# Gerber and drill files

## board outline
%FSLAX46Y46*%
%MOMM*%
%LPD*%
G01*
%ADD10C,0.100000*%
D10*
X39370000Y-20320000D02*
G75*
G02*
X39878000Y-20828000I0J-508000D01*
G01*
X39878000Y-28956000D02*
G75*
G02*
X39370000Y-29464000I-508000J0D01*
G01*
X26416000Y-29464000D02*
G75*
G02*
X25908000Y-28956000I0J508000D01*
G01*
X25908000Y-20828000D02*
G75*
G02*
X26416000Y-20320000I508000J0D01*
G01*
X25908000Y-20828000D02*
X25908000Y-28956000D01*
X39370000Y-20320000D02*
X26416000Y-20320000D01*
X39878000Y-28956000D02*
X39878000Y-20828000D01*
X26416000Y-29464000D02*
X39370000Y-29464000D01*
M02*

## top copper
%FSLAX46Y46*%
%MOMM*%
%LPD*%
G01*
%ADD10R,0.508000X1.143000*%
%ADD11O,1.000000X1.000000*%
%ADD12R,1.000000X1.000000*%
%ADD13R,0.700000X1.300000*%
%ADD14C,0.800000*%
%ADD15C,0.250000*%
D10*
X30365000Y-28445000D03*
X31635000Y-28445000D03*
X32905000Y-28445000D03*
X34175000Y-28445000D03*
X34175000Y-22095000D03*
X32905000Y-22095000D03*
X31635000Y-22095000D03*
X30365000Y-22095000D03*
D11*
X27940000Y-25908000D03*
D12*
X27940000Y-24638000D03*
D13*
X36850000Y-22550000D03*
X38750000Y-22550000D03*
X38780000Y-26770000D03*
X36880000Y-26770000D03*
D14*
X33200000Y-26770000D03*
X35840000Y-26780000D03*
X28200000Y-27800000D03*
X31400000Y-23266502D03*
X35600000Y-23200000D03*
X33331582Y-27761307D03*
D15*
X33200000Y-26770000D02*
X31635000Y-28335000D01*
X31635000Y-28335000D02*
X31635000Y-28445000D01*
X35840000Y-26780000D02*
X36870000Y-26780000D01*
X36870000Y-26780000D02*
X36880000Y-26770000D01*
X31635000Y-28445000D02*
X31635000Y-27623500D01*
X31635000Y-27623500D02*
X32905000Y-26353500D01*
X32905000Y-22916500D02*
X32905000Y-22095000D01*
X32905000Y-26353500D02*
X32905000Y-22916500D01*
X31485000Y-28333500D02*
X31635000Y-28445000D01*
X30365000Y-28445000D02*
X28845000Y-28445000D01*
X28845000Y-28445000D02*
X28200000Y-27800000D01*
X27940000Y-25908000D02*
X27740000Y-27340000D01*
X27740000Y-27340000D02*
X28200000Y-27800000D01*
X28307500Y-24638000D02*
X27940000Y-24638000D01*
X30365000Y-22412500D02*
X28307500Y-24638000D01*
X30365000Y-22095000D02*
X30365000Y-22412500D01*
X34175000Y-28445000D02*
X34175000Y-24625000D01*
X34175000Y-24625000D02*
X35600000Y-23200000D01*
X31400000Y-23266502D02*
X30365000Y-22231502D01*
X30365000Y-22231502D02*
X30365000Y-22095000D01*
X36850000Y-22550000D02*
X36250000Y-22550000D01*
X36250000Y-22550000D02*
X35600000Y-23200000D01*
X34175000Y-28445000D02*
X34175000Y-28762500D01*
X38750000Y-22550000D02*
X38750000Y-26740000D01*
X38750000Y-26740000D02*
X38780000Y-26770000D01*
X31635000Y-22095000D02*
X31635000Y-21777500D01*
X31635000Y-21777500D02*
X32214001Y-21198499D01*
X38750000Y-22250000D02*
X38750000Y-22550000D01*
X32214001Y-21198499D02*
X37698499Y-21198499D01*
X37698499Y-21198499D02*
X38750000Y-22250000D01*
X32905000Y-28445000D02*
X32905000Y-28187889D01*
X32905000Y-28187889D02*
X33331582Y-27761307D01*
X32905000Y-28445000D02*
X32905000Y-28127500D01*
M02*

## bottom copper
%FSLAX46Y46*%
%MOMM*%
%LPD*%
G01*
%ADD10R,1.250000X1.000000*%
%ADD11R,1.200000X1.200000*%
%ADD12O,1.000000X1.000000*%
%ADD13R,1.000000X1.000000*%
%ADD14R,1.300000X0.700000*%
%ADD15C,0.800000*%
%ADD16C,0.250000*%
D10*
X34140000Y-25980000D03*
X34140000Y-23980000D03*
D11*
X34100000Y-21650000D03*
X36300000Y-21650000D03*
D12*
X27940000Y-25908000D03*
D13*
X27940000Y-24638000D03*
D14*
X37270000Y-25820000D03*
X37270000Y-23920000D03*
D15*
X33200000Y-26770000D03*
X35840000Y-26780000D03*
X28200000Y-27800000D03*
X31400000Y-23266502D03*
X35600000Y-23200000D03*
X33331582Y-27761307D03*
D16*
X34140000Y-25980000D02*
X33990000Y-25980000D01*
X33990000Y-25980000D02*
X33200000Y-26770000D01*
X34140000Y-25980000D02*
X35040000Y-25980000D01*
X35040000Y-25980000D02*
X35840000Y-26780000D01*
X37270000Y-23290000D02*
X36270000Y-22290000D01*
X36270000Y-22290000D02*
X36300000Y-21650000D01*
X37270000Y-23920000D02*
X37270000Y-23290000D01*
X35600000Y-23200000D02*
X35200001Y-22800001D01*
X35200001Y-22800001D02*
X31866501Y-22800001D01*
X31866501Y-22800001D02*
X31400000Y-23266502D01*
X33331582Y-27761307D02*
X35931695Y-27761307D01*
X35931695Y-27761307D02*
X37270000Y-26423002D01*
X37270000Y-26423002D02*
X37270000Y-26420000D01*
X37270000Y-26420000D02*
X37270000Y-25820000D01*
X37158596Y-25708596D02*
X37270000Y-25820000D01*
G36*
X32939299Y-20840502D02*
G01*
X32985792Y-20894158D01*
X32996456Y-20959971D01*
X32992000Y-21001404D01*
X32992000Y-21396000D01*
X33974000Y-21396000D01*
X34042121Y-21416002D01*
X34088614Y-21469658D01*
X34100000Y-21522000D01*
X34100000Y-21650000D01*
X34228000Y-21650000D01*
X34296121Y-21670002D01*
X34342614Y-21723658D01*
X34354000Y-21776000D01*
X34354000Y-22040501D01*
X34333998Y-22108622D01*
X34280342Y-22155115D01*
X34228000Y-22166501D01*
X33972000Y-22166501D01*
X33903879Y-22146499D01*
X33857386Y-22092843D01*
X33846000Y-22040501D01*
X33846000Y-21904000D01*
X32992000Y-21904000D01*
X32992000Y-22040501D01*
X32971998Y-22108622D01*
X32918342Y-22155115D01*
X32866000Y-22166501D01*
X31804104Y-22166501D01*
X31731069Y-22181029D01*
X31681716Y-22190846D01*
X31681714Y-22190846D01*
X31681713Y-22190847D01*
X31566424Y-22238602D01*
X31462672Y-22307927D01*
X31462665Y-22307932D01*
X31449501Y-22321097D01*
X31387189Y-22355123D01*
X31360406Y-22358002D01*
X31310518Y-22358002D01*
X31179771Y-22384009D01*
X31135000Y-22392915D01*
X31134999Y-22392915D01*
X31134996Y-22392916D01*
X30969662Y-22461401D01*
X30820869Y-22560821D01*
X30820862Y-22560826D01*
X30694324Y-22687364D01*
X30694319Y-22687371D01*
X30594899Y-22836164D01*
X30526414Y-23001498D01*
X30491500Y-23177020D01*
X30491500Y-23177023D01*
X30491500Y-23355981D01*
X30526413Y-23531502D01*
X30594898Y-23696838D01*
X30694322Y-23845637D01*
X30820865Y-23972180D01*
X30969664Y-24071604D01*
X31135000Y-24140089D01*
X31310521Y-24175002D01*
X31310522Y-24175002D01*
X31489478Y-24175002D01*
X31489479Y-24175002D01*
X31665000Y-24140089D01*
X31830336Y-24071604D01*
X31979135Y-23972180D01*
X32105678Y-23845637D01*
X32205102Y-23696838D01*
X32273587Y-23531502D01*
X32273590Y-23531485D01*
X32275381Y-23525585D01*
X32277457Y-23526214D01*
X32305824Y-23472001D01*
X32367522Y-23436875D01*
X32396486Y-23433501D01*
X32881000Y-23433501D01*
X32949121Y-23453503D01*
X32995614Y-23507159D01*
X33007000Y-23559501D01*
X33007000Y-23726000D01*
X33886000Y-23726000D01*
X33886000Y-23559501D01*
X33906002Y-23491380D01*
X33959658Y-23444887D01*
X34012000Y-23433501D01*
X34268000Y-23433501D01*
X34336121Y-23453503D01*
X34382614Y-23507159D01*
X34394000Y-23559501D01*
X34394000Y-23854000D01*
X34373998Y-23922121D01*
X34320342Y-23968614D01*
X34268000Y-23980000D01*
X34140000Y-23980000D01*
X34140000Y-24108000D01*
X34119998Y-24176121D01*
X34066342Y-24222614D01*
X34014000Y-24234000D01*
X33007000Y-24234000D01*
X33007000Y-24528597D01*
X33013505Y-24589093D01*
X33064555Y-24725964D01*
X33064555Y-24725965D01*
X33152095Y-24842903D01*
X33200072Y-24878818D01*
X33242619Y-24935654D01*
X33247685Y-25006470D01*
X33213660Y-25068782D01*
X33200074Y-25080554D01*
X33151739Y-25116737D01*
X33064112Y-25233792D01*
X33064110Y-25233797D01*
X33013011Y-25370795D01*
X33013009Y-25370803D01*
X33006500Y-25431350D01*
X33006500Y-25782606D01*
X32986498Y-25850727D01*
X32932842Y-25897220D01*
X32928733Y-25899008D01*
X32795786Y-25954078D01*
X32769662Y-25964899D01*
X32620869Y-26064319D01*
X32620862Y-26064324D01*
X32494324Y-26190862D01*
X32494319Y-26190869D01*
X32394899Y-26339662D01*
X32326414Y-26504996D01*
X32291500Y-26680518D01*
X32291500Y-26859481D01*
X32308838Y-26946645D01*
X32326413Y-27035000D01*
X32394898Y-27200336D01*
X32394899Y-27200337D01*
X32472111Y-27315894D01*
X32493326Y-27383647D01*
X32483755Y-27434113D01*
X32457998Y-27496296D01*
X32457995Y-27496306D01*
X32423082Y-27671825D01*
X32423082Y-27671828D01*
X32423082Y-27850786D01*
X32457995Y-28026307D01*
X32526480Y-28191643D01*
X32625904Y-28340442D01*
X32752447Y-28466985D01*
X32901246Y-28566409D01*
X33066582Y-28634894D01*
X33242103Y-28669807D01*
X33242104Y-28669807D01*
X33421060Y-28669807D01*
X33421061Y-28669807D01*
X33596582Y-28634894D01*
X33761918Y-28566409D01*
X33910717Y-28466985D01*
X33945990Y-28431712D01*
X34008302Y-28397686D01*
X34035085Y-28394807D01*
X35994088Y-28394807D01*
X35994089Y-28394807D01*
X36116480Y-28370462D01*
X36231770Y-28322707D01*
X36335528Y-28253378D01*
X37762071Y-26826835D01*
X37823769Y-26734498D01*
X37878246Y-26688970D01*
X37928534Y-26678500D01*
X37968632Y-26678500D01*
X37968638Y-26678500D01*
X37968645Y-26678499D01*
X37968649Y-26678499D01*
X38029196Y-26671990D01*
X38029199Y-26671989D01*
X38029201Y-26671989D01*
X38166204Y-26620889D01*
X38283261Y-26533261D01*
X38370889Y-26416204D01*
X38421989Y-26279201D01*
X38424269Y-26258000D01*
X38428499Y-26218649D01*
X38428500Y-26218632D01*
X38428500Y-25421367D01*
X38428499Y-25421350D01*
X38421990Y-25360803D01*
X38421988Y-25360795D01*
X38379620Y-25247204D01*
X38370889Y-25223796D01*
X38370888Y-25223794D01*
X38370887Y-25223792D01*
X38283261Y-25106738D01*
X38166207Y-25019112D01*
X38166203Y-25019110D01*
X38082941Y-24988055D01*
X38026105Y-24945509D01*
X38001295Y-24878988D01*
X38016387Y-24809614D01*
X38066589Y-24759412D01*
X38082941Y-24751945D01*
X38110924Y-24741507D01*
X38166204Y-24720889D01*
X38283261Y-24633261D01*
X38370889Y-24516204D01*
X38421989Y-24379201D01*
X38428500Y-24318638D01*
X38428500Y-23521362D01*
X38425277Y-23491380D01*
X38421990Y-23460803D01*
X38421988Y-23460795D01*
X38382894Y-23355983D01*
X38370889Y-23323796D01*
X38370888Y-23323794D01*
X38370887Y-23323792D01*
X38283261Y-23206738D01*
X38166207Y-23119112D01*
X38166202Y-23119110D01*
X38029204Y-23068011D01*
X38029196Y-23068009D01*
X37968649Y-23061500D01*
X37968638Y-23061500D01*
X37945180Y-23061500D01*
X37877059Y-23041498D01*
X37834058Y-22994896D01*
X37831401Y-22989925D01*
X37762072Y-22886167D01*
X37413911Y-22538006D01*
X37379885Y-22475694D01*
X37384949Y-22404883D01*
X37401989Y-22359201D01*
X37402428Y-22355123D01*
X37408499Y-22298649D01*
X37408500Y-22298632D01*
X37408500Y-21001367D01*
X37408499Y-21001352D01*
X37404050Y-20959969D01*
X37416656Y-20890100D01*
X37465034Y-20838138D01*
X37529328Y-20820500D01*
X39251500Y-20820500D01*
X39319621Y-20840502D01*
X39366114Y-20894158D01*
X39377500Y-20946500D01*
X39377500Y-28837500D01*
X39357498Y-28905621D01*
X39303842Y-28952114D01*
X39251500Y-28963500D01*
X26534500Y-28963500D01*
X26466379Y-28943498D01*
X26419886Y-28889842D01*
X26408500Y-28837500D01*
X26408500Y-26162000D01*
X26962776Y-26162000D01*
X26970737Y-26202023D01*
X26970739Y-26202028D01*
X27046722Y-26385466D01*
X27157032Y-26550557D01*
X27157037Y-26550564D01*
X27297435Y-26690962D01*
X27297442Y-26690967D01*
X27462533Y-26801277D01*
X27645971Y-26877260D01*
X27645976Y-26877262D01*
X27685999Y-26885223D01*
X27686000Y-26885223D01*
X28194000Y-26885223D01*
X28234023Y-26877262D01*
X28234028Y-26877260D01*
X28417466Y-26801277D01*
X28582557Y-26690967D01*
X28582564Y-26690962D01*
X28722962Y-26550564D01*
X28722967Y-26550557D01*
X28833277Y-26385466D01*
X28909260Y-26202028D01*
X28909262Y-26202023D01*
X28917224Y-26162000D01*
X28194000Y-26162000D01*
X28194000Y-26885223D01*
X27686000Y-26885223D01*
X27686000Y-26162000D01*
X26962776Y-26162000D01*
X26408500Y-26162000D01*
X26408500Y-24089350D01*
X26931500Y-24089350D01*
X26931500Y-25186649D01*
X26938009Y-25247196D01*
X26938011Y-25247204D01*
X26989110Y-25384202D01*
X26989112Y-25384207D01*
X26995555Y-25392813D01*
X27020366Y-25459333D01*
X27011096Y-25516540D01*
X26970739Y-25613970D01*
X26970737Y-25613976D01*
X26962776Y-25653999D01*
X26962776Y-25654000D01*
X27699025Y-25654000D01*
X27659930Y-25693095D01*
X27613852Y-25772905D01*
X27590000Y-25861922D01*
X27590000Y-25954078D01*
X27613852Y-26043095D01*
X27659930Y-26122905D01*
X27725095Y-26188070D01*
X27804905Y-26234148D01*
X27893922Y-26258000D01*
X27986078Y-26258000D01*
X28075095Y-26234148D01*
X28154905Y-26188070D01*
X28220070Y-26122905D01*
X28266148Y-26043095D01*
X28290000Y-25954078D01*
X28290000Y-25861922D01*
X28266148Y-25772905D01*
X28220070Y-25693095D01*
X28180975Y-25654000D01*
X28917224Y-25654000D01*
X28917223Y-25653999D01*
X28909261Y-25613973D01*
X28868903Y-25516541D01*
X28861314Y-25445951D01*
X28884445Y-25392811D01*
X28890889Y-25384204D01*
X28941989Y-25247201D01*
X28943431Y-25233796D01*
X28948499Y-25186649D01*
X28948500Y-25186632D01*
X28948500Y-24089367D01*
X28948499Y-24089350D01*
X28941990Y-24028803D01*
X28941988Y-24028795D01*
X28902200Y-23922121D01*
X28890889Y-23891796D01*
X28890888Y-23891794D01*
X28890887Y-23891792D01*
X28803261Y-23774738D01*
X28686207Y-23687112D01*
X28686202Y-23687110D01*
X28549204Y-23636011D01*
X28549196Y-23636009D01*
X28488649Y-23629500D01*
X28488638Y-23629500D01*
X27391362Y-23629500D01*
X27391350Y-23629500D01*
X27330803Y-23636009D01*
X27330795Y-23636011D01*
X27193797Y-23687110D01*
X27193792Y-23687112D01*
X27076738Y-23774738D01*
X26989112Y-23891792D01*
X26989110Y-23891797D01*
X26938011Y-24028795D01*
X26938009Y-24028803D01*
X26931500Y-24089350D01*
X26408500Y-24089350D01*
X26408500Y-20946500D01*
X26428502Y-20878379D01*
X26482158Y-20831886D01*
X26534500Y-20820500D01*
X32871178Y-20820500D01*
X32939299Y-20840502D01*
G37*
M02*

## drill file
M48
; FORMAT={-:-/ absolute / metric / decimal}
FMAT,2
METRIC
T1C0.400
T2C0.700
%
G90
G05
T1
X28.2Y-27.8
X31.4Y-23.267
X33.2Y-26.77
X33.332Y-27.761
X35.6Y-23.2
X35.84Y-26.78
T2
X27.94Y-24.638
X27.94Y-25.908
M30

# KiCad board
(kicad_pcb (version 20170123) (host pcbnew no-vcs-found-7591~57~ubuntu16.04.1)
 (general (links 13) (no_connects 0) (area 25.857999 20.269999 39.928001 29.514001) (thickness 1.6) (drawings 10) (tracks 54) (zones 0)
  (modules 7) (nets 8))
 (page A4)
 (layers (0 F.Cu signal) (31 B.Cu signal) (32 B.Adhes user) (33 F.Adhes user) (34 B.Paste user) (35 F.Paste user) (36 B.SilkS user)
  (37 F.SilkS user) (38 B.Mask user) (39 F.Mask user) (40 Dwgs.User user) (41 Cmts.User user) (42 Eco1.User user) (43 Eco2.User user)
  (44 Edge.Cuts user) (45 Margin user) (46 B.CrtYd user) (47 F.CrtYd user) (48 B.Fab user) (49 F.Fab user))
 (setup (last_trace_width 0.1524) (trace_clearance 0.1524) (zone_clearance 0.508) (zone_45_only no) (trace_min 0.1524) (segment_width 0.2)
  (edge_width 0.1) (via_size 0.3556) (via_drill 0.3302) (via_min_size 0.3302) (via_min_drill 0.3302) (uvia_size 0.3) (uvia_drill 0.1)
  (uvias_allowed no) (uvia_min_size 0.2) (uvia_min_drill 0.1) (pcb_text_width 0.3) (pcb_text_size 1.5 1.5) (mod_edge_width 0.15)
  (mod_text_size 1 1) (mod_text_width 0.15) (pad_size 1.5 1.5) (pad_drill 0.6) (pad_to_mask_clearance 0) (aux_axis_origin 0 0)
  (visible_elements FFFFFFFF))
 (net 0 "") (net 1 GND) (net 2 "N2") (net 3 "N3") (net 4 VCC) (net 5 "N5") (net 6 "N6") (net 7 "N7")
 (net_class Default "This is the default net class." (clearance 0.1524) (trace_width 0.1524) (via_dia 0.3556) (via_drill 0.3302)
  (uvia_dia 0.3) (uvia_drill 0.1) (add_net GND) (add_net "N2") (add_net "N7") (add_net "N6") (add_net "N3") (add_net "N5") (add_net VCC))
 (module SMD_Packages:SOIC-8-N (layer F.Cu) (at 32.27 25.27)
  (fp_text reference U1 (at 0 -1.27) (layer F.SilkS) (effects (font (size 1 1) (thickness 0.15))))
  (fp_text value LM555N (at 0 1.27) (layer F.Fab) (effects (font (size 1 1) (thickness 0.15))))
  (pad 1 smd rect (at -1.905 3.175) (size 0.508 1.143) (layers F.Cu F.Paste F.Mask) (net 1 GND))
  (pad 2 smd rect (at -0.635 3.175) (size 0.508 1.143) (layers F.Cu F.Paste F.Mask) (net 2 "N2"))
  (pad 3 smd rect (at 0.635 3.175) (size 0.508 1.143) (layers F.Cu F.Paste F.Mask) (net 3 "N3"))
  (pad 4 smd rect (at 1.905 3.175) (size 0.508 1.143) (layers F.Cu F.Paste F.Mask) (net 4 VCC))
  (pad 5 smd rect (at 1.905 -3.175) (size 0.508 1.143) (layers F.Cu F.Paste F.Mask) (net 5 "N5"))
  (pad 6 smd rect (at 0.635 -3.175) (size 0.508 1.143) (layers F.Cu F.Paste F.Mask) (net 2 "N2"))
  (pad 7 smd rect (at -0.635 -3.175) (size 0.508 1.143) (layers F.Cu F.Paste F.Mask) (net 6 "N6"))
  (pad 8 smd rect (at -1.905 -3.175) (size 0.508 1.143) (layers F.Cu F.Paste F.Mask) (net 4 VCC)))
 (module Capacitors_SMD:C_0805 (layer B.Cu) (at 34.14 24.98 270)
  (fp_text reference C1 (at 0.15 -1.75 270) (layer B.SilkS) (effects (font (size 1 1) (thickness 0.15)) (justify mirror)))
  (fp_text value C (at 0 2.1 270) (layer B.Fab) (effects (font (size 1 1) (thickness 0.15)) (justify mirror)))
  (pad 2 smd rect (at 1 0 270) (size 1 1.25) (layers B.Cu B.Paste B.Mask) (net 2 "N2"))
  (pad 1 smd rect (at -1 0 270) (size 1 1.25) (layers B.Cu B.Paste B.Mask) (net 1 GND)))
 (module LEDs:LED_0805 (layer B.Cu) (at 35.2 21.65)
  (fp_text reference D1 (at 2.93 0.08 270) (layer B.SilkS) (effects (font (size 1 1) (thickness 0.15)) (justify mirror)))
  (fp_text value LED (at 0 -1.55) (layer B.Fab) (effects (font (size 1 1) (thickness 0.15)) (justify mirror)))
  (pad 1 smd rect (at -1.1 0 180) (size 1.2 1.2) (layers B.Cu B.Paste B.Mask) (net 1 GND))
  (pad 2 smd rect (at 1.1 0 180) (size 1.2 1.2) (layers B.Cu B.Paste B.Mask) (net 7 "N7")))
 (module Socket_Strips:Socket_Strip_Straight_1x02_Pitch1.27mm (layer F.Cu) (at 27.94 24.638)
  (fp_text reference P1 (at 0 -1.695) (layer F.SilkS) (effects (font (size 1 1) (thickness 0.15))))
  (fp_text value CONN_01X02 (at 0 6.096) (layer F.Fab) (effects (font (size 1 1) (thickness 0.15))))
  (pad 2 thru_hole oval (at 0 1.27) (size 1 1) (drill 0.7) (layers *.Cu *.Mask) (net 1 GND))
  (pad 1 thru_hole rect (at 0 0) (size 1 1) (drill 0.7) (layers *.Cu *.Mask) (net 4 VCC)))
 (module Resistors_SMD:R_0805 (layer F.Cu) (at 37.8 22.55 180)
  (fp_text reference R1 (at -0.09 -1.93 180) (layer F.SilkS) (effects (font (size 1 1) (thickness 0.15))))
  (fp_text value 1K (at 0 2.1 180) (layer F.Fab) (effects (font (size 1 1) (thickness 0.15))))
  (pad 2 smd rect (at 0.95 0 180) (size 0.7 1.3) (layers F.Cu F.Paste F.Mask) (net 4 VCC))
  (pad 1 smd rect (at -0.95 0 180) (size 0.7 1.3) (layers F.Cu F.Paste F.Mask) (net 6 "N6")))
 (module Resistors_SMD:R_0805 (layer B.Cu) (at 37.27 24.87 270)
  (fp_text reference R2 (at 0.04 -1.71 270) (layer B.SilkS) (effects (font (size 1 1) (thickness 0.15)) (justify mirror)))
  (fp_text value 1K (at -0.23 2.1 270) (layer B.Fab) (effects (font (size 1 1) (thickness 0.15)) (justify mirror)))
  (pad 2 smd rect (at 0.95 0 270) (size 0.7 1.3) (layers B.Cu B.Paste B.Mask) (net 3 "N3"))
  (pad 1 smd rect (at -0.95 0 270) (size 0.7 1.3) (layers B.Cu B.Paste B.Mask) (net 7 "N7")))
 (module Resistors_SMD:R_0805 (layer F.Cu) (at 37.83 26.77 180)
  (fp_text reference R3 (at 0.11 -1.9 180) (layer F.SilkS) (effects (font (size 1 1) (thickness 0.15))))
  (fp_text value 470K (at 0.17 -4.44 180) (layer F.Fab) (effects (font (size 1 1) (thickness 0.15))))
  (pad 1 smd rect (at -0.95 0 180) (size 0.7 1.3) (layers F.Cu F.Paste F.Mask) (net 6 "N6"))
  (pad 2 smd rect (at 0.95 0 180) (size 0.7 1.3) (layers F.Cu F.Paste F.Mask) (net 2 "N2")))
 (gr_arc (start 39.37 20.828) (end 39.37 20.32) (angle 90) (layer Edge.Cuts) (width 0.1))
 (gr_arc (start 39.37 28.956) (end 39.878 28.956) (angle 90) (layer Edge.Cuts) (width 0.1))
 (gr_arc (start 26.416 28.956) (end 26.416 29.464) (angle 90) (layer Edge.Cuts) (width 0.1))
 (gr_arc (start 26.416 20.828) (end 25.908 20.828) (angle 90) (layer Edge.Cuts) (width 0.1))
 (gr_line (start 25.908 20.828) (end 25.908 28.956) (angle 90) (layer Edge.Cuts) (width 0.1))
 (gr_line (start 39.37 20.32) (end 26.416 20.32) (angle 90) (layer Edge.Cuts) (width 0.1))
 (gr_line (start 39.878 28.956) (end 39.878 20.828) (angle 90) (layer Edge.Cuts) (width 0.1))
 (gr_line (start 26.416 29.464) (end 39.37 29.464) (angle 90) (layer Edge.Cuts) (width 0.1))
 (segment (start 33.2 26.77) (end 31.635 28.335) (width 0.25) (layer F.Cu) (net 2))
 (segment (start 31.635 28.335) (end 31.635 28.445) (width 0.25) (layer F.Cu) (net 2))
 (segment (start 34.14 25.98) (end 33.99 25.98) (width 0.25) (layer B.Cu) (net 2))
 (segment (start 33.99 25.98) (end 33.2 26.77) (width 0.25) (layer B.Cu) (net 2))
 (via (at 33.2 26.77) (size 0.8) (drill 0.4) (layers F.Cu B.Cu) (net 2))
 (segment (start 35.84 26.78) (end 36.87 26.78) (width 0.25) (layer F.Cu) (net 2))
 (segment (start 36.87 26.78) (end 36.88 26.77) (width 0.25) (layer F.Cu) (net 2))
 (segment (start 34.14 25.98) (end 35.04 25.98) (width 0.25) (layer B.Cu) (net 2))
 (segment (start 35.04 25.98) (end 35.84 26.78) (width 0.25) (layer B.Cu) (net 2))
 (via (at 35.84 26.78) (size 0.8) (drill 0.4) (layers F.Cu B.Cu) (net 2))
 (segment (start 31.635 28.445) (end 31.635 27.6235) (width 0.25) (layer F.Cu) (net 2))
 (segment (start 31.635 27.6235) (end 32.905 26.3535) (width 0.25) (layer F.Cu) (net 2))
 (segment (start 32.905 22.9165) (end 32.905 22.095) (width 0.25) (layer F.Cu) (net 2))
 (segment (start 32.905 26.3535) (end 32.905 22.9165) (width 0.25) (layer F.Cu) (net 2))
 (segment (start 31.485 28.3335) (end 31.635 28.445) (width 0.25) (layer F.Cu) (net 2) (status 20))
 (segment (start 30.365 28.445) (end 28.845 28.445) (width 0.25) (layer F.Cu) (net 1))
 (segment (start 28.845 28.445) (end 28.2 27.8) (width 0.25) (layer F.Cu) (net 1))
 (segment (start 27.94 25.908) (end 27.74 27.34) (width 0.25) (layer F.Cu) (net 1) (status 10))
 (segment (start 27.74 27.34) (end 28.2 27.8) (width 0.25) (layer F.Cu) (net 1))
 (via (at 28.2 27.8) (size 0.8) (drill 0.4) (layers F.Cu B.Cu) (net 1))
 (segment (start 37.27 23.29) (end 36.27 22.29) (width 0.25) (layer B.Cu) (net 7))
 (segment (start 36.27 22.29) (end 36.3 21.65) (width 0.25) (layer B.Cu) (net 7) (status 20))
 (segment (start 37.27 23.92) (end 37.27 23.29) (width 0.25) (layer B.Cu) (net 7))
 (segment (start 28.3075 24.638) (end 27.94 24.638) (width 0.25) (layer F.Cu) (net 4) (status 30))
 (segment (start 30.365 22.4125) (end 28.3075 24.638) (width 0.25) (layer F.Cu) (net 4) (status 20))
 (segment (start 30.365 22.095) (end 30.365 22.4125) (width 0.25) (layer F.Cu) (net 4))
 (segment (start 34.175 28.445) (end 34.175 24.625) (width 0.25) (layer F.Cu) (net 4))
 (segment (start 34.175 24.625) (end 35.6 23.2) (width 0.25) (layer F.Cu) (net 4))
 (segment (start 31.4 23.266502) (end 30.365 22.231502) (width 0.25) (layer F.Cu) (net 4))
 (segment (start 30.365 22.231502) (end 30.365 22.095) (width 0.25) (layer F.Cu) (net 4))
 (segment (start 35.6 23.2) (end 35.200001 22.800001) (width 0.25) (layer B.Cu) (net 4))
 (segment (start 35.200001 22.800001) (end 31.866501 22.800001) (width 0.25) (layer B.Cu) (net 4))
 (segment (start 31.866501 22.800001) (end 31.4 23.266502) (width 0.25) (layer B.Cu) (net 4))
 (via (at 31.4 23.266502) (size 0.8) (drill 0.4) (layers F.Cu B.Cu) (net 4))
 (segment (start 36.85 22.55) (end 36.25 22.55) (width 0.25) (layer F.Cu) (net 4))
 (segment (start 36.25 22.55) (end 35.6 23.2) (width 0.25) (layer F.Cu) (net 4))
 (via (at 35.6 23.2) (size 0.8) (drill 0.4) (layers F.Cu B.Cu) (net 4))
 (segment (start 34.175 28.445) (end 34.175 28.7625) (width 0.25) (layer F.Cu) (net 4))
 (segment (start 38.75 22.55) (end 38.75 26.74) (width 0.25) (layer F.Cu) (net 6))
 (segment (start 38.75 26.74) (end 38.78 26.77) (width 0.25) (layer F.Cu) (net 6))
 (segment (start 31.635 22.095) (end 31.635 21.7775) (width 0.25) (layer F.Cu) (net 6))
 (segment (start 31.635 21.7775) (end 32.214001 21.198499) (width 0.25) (layer F.Cu) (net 6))
 (segment (start 38.75 22.25) (end 38.75 22.55) (width 0.25) (layer F.Cu) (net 6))
 (segment (start 32.214001 21.198499) (end 37.698499 21.198499) (width 0.25) (layer F.Cu) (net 6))
 (segment (start 37.698499 21.198499) (end 38.75 22.25) (width 0.25) (layer F.Cu) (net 6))
 (segment (start 33.331582 27.761307) (end 35.931695 27.761307) (width 0.25) (layer B.Cu) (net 3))
 (segment (start 35.931695 27.761307) (end 37.27 26.423002) (width 0.25) (layer B.Cu) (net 3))
 (segment (start 37.27 26.423002) (end 37.27 26.42) (width 0.25) (layer B.Cu) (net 3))
 (segment (start 37.27 26.42) (end 37.27 25.82) (width 0.25) (layer B.Cu) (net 3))
 (segment (start 32.905 28.445) (end 32.905 28.187889) (width 0.25) (layer F.Cu) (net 3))
 (segment (start 32.905 28.187889) (end 33.331582 27.761307) (width 0.25) (layer F.Cu) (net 3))
 (via (at 33.331582 27.761307) (size 0.8) (drill 0.4) (layers F.Cu B.Cu) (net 3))
 (segment (start 37.158596 25.708596) (end 37.27 25.82) (width 0.25) (layer B.Cu) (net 3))
 (segment (start 32.905 28.445) (end 32.905 28.1275) (width 0.25) (layer F.Cu) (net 3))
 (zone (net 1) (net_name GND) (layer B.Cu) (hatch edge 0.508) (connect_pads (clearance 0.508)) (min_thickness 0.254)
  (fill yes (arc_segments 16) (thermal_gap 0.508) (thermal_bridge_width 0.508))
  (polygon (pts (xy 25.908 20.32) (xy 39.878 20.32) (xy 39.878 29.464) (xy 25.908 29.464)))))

